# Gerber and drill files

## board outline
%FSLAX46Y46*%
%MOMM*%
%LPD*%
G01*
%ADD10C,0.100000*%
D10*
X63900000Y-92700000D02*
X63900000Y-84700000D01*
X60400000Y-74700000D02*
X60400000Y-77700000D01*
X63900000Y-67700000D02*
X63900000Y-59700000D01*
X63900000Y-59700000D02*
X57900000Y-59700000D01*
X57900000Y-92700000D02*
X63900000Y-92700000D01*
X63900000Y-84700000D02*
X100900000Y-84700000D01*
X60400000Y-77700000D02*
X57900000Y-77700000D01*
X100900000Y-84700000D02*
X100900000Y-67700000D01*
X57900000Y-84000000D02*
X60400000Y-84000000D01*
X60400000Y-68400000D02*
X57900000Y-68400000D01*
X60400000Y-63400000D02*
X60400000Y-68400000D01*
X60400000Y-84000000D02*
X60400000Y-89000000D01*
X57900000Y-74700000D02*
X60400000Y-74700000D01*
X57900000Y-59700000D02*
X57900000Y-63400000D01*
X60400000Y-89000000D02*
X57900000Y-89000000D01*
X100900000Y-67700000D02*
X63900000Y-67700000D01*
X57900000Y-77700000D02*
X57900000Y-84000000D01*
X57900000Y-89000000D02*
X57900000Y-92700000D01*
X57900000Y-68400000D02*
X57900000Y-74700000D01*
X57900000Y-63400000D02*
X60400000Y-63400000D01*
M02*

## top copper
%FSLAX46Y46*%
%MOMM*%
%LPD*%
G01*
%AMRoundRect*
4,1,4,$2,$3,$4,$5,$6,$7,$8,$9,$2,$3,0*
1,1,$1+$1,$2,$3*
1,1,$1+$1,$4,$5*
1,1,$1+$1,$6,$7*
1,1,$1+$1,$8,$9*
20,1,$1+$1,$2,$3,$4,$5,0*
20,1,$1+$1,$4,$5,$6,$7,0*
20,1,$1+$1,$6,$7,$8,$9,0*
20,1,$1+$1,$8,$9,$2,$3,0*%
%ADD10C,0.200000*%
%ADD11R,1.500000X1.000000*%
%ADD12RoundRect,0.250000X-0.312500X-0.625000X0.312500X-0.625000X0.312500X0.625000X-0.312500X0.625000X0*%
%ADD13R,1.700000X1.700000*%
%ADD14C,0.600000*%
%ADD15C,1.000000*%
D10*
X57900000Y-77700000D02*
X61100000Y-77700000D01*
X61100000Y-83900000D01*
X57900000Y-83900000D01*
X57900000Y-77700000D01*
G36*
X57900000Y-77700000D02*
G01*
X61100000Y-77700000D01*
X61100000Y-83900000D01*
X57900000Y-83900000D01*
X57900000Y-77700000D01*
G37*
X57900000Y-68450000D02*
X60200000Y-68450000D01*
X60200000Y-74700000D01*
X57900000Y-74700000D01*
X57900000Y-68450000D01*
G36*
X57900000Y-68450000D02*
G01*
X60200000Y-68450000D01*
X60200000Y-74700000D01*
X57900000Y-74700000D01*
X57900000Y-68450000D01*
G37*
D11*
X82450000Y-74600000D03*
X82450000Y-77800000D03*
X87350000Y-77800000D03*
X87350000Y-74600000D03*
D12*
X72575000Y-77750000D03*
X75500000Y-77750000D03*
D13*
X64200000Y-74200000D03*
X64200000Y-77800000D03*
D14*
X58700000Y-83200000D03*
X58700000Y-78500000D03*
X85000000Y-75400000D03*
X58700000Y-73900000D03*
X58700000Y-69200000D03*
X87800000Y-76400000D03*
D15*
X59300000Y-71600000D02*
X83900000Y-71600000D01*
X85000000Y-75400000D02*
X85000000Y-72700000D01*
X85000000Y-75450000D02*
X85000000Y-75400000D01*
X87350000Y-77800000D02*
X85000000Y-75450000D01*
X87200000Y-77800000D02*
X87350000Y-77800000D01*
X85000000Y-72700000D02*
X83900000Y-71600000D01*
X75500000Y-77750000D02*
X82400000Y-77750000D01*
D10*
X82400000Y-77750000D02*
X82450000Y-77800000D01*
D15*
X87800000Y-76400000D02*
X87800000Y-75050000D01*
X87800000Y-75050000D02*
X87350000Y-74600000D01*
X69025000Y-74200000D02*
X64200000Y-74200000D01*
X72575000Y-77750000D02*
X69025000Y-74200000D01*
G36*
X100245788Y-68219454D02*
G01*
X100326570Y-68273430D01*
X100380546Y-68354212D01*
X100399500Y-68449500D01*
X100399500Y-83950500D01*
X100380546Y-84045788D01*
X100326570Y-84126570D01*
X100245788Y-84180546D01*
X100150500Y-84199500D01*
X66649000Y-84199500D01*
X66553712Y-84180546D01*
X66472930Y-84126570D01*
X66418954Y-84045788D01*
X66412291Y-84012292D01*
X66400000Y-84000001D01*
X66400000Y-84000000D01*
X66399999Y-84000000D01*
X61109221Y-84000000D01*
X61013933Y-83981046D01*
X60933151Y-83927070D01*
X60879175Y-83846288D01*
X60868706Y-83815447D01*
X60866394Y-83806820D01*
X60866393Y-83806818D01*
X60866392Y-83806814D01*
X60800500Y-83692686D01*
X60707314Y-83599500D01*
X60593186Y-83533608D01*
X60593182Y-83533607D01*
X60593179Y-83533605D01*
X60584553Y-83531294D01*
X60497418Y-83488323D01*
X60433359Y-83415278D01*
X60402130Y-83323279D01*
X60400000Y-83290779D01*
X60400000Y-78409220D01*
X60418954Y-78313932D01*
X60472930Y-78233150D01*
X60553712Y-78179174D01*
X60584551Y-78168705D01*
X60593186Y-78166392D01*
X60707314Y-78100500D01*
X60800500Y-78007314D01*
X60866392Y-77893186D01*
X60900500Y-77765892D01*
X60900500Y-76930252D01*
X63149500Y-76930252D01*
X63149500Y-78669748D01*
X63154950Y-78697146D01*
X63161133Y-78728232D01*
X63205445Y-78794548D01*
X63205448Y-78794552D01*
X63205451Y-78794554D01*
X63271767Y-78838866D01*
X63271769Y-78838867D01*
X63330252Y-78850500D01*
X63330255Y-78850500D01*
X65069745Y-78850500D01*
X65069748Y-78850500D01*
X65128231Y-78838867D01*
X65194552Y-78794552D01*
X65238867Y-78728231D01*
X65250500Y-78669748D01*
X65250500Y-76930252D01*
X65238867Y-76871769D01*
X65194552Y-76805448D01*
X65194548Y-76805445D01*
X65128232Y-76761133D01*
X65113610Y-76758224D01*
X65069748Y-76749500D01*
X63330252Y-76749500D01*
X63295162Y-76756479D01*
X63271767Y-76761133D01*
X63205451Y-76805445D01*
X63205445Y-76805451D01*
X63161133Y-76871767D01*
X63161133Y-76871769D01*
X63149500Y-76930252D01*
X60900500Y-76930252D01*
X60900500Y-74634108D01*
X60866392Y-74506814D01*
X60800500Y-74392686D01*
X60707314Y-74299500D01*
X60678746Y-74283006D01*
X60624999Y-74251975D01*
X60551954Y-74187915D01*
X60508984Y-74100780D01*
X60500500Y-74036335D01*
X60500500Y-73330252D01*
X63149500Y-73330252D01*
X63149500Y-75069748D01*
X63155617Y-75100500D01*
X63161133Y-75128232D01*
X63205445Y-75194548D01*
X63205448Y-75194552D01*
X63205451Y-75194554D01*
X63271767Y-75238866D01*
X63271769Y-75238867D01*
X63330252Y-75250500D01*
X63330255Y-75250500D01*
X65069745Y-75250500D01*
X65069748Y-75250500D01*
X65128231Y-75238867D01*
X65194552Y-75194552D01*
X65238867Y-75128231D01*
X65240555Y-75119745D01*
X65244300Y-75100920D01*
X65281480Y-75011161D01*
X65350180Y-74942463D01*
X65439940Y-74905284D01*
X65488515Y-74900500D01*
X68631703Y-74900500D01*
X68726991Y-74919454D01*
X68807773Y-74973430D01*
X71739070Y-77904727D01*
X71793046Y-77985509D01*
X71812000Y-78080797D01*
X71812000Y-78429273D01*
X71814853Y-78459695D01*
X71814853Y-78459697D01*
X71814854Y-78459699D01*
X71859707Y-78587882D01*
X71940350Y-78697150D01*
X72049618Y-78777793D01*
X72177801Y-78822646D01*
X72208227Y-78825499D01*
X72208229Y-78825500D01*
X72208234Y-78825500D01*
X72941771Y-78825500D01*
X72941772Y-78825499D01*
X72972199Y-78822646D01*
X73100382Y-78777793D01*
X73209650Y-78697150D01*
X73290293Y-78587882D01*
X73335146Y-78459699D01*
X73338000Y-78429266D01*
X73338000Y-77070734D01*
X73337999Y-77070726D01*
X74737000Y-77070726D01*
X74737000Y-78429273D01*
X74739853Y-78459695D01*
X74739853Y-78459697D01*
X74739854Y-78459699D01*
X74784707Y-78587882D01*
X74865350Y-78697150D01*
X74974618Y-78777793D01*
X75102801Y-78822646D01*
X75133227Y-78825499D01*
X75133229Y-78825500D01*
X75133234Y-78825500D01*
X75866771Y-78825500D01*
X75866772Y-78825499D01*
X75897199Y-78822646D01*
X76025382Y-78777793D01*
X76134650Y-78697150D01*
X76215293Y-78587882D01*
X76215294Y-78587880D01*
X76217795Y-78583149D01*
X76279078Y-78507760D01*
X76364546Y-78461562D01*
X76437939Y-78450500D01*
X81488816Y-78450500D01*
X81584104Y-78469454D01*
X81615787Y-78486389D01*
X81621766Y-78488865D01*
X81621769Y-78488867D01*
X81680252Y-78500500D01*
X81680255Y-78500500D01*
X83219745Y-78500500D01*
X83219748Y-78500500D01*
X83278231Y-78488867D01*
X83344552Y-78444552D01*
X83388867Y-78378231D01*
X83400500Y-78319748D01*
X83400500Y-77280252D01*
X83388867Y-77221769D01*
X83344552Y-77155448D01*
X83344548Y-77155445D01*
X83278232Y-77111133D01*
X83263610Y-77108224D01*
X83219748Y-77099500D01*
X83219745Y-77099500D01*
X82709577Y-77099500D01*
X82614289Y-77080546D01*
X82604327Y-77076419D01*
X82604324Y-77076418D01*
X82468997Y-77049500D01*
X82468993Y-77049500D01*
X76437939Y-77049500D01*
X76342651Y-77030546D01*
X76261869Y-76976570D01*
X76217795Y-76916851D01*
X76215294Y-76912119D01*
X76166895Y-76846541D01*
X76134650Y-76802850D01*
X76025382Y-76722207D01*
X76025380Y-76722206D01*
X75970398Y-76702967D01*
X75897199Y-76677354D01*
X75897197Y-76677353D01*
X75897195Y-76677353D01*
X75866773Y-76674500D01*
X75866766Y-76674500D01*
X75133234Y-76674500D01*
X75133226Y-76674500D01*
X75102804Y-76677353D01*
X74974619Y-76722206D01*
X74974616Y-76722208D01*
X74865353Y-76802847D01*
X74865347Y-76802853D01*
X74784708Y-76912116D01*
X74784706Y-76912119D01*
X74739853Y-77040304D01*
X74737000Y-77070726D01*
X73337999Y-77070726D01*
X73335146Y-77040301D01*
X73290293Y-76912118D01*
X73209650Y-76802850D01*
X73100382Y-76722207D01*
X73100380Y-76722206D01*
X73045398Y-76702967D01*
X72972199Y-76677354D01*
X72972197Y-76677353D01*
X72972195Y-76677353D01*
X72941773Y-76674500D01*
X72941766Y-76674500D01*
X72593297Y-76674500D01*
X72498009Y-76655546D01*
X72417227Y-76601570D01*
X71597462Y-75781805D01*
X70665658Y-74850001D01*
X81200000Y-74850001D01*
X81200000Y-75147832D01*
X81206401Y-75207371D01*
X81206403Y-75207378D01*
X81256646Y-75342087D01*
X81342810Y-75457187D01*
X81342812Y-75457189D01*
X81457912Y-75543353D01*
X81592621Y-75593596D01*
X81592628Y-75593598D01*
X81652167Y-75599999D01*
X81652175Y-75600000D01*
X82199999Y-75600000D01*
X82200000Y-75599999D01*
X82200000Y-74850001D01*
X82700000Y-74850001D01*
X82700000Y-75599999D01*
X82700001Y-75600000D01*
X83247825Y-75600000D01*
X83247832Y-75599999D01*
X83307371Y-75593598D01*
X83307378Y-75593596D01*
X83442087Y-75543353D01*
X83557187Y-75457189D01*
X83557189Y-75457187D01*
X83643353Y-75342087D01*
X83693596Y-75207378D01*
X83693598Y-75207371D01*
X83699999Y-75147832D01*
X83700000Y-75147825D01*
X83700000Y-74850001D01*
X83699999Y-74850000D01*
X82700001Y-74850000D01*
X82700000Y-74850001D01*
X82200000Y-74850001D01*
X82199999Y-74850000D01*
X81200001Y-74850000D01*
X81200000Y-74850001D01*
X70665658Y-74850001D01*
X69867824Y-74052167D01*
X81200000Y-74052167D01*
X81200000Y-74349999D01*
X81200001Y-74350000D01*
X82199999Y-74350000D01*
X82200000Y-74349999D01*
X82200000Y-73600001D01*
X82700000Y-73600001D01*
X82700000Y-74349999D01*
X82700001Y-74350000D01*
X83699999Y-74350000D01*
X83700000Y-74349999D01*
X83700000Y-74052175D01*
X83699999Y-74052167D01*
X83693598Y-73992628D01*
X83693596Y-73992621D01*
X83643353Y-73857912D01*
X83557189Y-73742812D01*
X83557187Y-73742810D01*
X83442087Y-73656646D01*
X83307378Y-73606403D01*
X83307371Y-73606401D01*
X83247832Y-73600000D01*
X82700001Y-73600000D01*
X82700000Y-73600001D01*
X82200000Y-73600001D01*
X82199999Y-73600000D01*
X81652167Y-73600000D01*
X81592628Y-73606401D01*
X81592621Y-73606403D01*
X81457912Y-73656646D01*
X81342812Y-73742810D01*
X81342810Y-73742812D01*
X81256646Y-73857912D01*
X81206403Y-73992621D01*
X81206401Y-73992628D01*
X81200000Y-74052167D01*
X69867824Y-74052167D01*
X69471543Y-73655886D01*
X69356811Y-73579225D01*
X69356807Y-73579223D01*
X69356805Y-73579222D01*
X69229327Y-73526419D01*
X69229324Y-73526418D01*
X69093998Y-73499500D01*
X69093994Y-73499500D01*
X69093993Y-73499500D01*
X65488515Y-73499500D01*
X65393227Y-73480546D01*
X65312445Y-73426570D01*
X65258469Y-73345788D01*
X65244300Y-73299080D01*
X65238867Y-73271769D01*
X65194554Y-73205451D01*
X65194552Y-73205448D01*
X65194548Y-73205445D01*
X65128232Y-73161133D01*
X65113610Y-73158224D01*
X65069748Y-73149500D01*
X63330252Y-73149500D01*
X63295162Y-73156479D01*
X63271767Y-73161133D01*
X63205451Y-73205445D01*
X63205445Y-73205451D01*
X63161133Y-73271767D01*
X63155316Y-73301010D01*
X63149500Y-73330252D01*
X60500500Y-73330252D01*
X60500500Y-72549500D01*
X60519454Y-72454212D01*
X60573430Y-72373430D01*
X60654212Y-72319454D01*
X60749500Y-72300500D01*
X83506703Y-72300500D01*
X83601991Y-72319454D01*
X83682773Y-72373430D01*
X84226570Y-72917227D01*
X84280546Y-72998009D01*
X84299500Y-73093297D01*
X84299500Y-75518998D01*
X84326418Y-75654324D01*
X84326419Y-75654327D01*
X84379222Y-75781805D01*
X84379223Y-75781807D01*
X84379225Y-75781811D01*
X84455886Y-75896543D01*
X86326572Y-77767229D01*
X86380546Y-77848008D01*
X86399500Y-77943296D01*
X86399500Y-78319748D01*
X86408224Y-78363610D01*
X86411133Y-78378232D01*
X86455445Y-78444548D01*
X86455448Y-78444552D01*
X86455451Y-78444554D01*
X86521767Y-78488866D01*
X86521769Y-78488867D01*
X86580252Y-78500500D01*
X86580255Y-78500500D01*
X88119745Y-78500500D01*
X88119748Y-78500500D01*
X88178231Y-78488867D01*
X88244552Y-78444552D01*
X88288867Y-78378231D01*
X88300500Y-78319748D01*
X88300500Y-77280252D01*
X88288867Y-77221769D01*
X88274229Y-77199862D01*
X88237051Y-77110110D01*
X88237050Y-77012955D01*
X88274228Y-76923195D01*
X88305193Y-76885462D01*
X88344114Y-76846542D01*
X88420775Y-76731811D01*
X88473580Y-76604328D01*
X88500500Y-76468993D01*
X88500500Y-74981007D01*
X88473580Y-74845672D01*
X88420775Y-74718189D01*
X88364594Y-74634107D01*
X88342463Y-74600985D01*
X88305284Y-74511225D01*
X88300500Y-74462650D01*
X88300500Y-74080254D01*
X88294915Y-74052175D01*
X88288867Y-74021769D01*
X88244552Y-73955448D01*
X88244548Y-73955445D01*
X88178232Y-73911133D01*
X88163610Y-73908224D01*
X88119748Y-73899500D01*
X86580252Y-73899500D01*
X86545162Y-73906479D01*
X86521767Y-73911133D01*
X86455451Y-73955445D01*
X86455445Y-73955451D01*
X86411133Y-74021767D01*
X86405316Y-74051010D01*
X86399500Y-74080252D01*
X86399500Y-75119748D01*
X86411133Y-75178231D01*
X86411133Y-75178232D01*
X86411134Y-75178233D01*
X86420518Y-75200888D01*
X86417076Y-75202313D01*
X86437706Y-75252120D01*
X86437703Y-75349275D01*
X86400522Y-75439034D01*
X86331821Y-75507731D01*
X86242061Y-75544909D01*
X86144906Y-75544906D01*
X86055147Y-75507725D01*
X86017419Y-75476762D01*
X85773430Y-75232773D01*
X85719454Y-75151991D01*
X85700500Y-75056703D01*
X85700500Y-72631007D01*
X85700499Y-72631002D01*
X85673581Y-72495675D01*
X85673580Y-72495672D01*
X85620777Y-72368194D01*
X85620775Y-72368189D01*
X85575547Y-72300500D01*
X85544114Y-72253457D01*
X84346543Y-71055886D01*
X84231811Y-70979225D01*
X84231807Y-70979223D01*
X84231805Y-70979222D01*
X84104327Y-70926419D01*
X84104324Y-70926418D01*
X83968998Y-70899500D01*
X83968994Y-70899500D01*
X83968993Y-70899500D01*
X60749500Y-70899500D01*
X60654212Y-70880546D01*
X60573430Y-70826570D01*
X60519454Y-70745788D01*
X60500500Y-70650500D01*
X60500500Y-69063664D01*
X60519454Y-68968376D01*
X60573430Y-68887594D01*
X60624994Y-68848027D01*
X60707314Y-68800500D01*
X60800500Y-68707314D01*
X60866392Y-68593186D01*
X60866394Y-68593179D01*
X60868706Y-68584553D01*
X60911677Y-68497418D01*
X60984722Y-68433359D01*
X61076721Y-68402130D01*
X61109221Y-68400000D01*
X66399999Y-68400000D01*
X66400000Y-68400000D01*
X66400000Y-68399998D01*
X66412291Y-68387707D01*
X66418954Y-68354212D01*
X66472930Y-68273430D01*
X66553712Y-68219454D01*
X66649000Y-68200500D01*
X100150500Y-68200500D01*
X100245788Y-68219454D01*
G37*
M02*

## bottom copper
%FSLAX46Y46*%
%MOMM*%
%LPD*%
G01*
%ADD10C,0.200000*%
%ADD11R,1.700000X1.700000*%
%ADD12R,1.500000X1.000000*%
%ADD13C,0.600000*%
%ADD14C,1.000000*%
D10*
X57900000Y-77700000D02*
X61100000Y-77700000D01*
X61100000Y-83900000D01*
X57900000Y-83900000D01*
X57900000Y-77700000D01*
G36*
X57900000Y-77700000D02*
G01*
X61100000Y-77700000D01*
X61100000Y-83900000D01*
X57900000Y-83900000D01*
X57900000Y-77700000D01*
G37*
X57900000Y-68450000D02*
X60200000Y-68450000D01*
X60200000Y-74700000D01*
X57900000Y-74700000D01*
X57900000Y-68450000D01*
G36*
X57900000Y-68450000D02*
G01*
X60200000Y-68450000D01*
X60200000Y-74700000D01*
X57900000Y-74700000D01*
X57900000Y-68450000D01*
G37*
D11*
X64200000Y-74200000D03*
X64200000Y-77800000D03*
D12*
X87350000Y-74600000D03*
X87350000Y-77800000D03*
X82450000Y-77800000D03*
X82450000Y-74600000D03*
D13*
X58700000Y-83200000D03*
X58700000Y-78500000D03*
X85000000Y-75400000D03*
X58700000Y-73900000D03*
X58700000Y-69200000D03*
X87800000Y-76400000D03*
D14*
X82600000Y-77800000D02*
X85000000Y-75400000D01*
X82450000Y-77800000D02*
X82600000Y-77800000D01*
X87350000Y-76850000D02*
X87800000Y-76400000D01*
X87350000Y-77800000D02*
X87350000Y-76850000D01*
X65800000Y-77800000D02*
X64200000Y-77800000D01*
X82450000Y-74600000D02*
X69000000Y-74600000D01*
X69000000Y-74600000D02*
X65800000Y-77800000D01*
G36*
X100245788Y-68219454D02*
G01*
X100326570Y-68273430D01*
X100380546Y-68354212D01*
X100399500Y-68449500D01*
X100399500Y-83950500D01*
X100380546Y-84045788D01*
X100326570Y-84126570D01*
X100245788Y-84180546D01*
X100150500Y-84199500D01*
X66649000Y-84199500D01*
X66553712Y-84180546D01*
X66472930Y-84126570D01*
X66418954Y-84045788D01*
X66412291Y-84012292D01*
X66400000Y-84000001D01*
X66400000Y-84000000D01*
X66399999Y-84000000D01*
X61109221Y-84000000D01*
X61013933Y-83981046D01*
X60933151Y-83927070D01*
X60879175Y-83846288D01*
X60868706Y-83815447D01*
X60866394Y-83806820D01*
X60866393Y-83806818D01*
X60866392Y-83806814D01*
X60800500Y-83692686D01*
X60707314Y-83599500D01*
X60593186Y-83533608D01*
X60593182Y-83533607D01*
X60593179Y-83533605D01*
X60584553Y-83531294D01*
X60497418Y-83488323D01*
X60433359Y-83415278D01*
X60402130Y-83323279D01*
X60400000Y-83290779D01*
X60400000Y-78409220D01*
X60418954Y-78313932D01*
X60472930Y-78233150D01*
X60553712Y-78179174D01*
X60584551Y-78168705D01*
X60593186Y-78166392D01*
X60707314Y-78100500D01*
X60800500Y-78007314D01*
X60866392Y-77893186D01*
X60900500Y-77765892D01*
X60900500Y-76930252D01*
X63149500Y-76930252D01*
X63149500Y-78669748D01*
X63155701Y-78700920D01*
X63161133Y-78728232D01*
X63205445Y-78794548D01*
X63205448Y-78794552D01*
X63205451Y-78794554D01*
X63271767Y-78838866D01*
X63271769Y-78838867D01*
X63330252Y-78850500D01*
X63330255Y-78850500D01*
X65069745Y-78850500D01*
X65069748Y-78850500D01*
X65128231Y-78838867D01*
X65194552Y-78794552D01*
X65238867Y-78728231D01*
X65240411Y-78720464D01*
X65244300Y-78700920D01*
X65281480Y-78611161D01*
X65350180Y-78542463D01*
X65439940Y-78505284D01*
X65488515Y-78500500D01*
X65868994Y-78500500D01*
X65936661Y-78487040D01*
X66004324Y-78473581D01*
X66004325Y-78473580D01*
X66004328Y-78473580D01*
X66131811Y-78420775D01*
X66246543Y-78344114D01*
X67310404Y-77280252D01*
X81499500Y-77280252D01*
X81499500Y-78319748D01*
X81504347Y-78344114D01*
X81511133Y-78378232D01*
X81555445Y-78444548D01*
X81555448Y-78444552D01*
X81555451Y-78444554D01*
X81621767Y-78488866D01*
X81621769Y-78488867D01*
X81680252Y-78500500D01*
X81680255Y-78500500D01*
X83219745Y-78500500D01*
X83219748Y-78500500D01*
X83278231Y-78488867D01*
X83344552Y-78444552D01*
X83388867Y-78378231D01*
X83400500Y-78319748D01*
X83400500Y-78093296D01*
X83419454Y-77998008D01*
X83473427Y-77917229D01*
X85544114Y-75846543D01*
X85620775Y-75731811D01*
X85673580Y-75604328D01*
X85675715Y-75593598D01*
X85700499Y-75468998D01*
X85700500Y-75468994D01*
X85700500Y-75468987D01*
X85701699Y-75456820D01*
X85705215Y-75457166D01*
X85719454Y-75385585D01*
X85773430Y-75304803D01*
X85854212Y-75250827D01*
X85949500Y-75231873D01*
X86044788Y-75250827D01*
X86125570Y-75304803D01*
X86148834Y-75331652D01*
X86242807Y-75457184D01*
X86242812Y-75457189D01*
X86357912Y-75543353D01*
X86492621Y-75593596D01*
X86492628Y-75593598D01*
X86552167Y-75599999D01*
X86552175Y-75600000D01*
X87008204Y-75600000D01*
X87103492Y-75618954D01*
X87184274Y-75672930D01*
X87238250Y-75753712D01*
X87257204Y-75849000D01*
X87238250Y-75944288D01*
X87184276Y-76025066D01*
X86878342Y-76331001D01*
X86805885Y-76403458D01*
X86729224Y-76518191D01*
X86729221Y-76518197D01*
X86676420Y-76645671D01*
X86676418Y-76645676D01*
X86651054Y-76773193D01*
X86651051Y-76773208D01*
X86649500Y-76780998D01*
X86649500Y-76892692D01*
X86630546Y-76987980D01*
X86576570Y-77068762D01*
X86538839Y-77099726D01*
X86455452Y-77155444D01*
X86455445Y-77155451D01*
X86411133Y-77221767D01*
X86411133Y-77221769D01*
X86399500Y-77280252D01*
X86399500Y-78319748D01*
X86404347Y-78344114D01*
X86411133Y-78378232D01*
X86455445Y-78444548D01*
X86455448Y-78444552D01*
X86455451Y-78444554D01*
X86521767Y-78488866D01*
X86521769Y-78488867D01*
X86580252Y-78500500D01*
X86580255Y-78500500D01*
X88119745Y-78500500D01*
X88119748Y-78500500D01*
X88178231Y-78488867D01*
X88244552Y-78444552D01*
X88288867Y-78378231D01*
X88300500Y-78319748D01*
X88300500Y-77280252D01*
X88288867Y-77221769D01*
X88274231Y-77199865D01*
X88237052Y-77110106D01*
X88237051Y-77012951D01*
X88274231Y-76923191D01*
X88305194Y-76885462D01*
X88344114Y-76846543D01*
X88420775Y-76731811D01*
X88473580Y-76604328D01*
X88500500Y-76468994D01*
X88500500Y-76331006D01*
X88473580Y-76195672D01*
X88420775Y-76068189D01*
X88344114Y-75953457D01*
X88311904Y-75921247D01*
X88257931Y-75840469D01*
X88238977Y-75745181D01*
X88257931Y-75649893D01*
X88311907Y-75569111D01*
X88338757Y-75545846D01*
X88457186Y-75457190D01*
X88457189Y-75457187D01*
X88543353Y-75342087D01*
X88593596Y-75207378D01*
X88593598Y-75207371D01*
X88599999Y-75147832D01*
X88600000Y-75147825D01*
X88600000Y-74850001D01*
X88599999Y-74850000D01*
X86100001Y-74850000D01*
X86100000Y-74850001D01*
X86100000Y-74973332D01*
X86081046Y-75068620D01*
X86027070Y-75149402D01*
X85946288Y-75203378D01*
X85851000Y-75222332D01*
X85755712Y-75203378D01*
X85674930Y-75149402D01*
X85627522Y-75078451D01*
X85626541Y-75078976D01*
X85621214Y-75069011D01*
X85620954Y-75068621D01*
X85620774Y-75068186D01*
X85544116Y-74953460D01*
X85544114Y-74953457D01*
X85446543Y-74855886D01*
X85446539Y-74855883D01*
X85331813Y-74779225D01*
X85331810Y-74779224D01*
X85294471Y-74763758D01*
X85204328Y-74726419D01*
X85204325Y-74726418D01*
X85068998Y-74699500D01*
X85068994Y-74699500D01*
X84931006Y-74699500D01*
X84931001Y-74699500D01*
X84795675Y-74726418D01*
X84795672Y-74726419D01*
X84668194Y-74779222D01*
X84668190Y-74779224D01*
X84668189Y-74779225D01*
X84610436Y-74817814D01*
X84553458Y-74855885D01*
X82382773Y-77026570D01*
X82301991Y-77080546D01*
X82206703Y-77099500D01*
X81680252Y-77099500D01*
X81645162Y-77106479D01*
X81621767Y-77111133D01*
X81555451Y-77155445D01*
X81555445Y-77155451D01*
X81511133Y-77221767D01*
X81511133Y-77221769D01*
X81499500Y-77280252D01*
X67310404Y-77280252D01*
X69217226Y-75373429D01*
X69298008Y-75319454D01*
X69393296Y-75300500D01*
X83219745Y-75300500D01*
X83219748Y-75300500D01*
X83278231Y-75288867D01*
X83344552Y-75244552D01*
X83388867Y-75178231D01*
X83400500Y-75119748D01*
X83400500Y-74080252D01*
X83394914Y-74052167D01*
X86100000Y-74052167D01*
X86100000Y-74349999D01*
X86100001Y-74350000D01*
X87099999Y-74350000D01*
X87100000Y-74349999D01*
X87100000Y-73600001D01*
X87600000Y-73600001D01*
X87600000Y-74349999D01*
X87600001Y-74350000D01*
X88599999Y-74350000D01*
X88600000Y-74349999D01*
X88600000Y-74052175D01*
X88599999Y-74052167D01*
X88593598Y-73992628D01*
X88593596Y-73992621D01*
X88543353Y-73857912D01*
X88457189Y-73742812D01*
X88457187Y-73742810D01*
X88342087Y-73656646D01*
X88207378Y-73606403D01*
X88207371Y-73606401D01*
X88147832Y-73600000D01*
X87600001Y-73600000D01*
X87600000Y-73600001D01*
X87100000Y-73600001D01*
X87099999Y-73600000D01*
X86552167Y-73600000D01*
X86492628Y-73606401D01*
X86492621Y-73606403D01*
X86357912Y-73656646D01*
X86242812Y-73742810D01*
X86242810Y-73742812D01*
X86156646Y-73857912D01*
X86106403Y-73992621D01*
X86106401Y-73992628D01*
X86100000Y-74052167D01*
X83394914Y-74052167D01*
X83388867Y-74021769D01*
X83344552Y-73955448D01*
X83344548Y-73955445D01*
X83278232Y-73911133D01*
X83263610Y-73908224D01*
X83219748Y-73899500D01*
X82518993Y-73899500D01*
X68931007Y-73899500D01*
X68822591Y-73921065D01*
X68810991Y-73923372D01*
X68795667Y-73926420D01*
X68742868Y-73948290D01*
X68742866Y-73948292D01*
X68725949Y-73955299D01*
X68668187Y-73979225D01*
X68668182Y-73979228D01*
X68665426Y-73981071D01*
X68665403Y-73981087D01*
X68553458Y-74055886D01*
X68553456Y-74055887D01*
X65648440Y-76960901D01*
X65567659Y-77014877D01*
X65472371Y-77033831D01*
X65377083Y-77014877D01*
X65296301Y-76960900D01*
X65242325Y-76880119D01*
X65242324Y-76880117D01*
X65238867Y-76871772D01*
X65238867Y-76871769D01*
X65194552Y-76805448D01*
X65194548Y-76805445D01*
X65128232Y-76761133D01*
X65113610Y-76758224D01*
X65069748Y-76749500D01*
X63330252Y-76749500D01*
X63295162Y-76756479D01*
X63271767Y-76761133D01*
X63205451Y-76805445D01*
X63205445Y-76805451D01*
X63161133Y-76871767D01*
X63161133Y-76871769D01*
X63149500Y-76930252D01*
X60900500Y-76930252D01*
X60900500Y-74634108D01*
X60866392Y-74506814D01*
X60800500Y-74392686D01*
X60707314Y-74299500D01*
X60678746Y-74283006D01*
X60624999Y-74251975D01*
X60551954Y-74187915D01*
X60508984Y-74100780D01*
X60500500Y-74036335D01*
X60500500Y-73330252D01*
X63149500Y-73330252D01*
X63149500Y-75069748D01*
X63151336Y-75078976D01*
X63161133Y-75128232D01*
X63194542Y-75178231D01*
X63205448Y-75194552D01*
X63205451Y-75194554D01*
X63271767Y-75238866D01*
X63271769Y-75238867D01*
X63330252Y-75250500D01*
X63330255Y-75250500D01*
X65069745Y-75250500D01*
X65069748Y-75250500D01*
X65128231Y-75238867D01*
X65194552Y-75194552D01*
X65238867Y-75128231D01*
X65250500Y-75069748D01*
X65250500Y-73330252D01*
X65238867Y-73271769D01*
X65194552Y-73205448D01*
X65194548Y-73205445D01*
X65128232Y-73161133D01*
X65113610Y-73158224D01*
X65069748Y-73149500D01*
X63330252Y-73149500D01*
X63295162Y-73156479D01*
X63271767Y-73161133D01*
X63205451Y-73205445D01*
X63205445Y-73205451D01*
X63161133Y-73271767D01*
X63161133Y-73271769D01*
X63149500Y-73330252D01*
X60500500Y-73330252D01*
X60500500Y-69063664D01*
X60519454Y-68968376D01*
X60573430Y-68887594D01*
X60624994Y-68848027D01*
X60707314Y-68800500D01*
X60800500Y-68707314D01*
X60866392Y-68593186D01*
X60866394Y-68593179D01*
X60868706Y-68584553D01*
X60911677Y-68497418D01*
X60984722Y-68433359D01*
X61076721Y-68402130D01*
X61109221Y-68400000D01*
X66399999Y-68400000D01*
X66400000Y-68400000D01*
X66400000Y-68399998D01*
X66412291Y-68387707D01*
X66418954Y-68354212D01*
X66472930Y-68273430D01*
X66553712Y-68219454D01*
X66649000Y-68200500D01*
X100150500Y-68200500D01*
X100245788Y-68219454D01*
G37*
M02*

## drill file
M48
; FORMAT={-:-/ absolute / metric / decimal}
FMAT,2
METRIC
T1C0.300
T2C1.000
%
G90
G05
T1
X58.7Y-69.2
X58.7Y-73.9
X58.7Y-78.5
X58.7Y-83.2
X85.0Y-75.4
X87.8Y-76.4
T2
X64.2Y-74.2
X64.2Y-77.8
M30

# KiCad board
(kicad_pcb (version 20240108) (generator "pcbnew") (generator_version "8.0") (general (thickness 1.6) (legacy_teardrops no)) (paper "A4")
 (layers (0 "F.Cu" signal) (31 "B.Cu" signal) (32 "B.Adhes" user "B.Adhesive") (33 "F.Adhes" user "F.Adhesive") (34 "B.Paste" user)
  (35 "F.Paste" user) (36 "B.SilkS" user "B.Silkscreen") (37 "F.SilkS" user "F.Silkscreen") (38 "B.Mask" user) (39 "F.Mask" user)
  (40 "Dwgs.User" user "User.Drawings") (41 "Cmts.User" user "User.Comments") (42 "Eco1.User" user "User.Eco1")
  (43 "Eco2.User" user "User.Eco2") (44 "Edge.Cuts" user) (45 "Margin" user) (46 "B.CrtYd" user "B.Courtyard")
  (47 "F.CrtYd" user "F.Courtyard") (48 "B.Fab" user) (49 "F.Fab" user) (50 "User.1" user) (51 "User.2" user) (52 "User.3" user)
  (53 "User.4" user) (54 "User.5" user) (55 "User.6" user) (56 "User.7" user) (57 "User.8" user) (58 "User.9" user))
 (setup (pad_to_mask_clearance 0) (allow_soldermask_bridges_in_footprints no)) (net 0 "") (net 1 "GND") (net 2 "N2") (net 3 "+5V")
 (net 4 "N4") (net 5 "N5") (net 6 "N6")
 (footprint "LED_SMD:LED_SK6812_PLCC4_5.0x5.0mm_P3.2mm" (layer "F.Cu") (at 84.9 76.2 180)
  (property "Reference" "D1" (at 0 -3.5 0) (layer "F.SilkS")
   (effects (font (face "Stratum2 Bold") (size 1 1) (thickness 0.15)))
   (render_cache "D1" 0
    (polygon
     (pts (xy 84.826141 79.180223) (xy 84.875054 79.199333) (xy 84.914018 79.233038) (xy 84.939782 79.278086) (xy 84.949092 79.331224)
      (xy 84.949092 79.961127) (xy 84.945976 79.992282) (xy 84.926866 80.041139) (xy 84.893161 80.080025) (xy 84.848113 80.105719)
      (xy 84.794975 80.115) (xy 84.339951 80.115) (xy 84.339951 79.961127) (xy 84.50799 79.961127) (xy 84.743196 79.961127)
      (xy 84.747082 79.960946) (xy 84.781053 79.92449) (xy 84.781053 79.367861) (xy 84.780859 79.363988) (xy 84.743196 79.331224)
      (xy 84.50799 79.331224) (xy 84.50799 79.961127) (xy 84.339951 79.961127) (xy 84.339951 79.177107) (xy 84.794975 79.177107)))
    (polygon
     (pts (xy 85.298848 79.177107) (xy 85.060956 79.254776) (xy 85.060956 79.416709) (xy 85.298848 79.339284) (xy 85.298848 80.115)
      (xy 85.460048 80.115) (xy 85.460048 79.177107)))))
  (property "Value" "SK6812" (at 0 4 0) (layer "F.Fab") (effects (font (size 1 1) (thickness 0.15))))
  (pad "1" smd rect (at 2.45 1.6 180) (size 1.5 1) (layers "F.Cu" "F.Paste" "F.Mask") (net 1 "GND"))
  (pad "2" smd rect (at 2.45 -1.6 180) (size 1.5 1) (layers "F.Cu" "F.Paste" "F.Mask") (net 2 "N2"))
  (pad "3" smd rect (at -2.45 -1.6 180) (size 1.5 1) (layers "F.Cu" "F.Paste" "F.Mask") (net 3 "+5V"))
  (pad "4" smd rect (at -2.45 1.6 180) (size 1.5 1) (layers "F.Cu" "F.Paste" "F.Mask") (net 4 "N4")))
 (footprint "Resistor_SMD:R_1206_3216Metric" (layer "F.Cu") (at 74.0375 77.75)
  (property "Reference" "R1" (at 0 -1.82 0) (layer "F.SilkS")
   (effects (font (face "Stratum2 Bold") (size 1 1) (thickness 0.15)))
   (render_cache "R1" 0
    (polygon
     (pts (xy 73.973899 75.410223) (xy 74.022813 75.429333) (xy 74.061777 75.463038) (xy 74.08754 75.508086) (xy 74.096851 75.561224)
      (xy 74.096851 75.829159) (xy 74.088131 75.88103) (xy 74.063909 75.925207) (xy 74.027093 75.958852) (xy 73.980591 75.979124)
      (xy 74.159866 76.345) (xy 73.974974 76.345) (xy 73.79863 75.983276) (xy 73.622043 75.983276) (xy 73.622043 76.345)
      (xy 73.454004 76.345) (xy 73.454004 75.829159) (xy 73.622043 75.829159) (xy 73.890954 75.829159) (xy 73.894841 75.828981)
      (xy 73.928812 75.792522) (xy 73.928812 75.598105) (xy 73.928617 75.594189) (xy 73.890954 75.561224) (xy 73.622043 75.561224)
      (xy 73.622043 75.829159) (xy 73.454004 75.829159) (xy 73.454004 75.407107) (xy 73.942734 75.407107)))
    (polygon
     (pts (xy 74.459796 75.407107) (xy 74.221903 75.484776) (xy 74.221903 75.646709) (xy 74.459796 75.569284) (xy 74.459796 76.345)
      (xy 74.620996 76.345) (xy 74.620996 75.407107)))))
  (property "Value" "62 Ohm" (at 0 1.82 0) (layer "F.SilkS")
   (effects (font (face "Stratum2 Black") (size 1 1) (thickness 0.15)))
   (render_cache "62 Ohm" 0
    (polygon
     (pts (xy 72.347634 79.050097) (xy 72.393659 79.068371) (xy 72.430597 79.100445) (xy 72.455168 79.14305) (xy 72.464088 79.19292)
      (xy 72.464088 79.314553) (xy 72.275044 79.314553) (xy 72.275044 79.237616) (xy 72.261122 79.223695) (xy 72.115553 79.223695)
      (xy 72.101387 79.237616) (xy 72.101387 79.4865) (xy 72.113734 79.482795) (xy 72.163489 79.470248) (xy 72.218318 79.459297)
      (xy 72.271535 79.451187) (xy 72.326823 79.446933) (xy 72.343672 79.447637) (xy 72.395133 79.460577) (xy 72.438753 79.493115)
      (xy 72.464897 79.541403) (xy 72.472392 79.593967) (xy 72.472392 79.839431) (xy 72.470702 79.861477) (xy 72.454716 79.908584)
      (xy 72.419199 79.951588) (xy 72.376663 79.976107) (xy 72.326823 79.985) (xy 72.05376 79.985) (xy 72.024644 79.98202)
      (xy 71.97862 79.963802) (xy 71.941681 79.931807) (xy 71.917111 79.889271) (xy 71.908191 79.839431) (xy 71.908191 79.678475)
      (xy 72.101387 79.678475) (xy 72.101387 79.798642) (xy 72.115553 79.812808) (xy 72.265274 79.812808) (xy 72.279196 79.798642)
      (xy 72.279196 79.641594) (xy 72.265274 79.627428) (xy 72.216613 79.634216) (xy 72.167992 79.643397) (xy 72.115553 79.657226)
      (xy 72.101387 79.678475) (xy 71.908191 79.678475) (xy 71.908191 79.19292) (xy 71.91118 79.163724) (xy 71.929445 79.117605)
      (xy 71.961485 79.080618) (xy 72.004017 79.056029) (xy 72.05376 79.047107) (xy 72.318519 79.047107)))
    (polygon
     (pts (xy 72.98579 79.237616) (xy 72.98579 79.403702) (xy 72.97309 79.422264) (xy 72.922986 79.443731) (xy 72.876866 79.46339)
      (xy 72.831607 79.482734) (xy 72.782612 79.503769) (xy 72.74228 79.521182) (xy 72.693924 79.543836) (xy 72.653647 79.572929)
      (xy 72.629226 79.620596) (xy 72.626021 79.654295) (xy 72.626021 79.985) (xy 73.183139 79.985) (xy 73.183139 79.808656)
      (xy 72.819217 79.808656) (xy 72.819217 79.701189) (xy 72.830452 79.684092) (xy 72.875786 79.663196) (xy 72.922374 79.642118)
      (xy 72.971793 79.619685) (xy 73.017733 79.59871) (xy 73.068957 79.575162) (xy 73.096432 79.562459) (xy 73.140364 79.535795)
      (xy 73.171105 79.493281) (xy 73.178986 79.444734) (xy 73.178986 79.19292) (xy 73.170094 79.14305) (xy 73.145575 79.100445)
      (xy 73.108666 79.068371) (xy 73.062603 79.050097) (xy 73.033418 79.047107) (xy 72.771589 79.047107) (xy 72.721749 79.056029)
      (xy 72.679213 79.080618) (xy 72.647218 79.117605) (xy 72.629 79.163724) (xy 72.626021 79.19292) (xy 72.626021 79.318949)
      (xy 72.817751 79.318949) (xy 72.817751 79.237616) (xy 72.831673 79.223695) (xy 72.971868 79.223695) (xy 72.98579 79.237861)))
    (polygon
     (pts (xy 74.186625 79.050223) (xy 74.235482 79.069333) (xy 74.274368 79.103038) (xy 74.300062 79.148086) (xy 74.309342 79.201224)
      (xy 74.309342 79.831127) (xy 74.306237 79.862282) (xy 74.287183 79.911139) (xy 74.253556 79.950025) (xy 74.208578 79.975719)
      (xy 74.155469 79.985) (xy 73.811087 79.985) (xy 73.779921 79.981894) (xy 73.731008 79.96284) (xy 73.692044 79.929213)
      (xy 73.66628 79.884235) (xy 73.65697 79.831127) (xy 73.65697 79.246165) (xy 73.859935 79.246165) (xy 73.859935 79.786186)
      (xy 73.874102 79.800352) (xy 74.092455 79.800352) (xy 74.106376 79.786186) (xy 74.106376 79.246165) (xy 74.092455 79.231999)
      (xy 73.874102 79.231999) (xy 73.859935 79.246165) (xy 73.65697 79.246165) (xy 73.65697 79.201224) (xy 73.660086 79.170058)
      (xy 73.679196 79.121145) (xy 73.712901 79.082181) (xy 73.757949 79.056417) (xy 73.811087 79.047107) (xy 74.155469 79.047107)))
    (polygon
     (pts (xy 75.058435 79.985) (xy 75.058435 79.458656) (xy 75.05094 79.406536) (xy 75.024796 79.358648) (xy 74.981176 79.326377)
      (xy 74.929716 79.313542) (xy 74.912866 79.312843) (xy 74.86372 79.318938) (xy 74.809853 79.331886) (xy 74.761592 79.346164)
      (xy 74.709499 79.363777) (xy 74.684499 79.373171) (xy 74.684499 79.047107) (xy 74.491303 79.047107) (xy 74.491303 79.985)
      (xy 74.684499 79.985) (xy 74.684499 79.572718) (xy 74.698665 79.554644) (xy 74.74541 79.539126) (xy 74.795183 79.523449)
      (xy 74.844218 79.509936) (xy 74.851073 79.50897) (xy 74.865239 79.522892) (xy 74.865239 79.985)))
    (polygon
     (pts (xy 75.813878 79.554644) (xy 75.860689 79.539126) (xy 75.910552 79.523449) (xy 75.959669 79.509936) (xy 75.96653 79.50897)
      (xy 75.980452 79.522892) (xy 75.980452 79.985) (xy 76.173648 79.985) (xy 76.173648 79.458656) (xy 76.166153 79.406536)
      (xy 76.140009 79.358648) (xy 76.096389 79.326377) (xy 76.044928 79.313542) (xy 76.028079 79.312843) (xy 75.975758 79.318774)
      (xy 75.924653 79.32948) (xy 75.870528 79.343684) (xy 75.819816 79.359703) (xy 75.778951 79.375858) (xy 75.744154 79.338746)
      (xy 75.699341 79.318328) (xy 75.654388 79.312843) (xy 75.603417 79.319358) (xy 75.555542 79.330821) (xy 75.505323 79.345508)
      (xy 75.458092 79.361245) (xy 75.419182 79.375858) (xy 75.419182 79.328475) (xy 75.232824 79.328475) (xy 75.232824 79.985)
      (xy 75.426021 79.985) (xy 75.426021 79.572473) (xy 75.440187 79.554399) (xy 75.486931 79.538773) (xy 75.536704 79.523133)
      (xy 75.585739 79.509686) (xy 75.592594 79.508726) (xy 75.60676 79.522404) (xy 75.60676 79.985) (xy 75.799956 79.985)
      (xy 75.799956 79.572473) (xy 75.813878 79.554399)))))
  (pad "1" smd roundrect (at -1.4625 0) (size 1.125 1.75) (layers "F.Cu" "F.Paste" "F.Mask") (roundrect_rratio 0.222222) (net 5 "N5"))
  (pad "2" smd roundrect (at 1.4625 0) (size 1.125 1.75) (layers "F.Cu" "F.Paste" "F.Mask") (roundrect_rratio 0.222222) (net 2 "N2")))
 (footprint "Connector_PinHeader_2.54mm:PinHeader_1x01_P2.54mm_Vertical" (layer "F.Cu") (at 64.2 74.2)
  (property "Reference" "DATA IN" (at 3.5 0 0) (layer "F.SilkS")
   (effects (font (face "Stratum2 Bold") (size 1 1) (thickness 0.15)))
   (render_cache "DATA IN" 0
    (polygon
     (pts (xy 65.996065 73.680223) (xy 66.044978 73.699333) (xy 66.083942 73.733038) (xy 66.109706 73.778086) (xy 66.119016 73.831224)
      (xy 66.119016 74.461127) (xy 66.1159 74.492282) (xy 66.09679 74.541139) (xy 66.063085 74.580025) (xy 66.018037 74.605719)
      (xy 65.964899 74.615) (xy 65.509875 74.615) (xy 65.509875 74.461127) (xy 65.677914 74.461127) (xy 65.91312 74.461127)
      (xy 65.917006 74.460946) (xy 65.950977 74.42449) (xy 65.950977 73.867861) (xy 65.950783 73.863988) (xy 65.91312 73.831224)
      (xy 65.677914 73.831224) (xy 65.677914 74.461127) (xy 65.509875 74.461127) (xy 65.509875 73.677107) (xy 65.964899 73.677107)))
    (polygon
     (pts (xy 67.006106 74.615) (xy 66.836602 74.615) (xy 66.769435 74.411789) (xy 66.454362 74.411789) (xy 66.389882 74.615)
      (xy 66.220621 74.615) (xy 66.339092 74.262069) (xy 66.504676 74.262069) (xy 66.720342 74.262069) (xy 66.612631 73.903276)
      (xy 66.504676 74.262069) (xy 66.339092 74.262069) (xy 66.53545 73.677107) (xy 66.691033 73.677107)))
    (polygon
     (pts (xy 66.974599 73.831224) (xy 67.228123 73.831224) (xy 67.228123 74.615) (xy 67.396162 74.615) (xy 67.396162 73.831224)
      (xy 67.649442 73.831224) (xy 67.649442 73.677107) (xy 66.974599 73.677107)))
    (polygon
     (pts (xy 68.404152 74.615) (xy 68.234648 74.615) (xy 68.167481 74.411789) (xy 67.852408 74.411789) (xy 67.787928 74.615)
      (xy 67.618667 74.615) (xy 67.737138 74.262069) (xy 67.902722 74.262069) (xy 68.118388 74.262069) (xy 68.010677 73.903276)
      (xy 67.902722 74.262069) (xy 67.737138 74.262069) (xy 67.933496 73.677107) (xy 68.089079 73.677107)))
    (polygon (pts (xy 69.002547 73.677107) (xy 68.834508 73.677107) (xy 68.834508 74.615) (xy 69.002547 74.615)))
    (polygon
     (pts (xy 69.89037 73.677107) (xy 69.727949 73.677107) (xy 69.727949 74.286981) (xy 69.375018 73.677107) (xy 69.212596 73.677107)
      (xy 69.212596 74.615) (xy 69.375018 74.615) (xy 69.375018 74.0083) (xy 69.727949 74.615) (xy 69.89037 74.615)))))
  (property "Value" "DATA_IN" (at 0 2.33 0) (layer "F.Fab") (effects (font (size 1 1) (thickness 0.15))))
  (pad "1" thru_hole rect (at 0 0) (size 1.7 1.7) (drill 1) (layers "*.Cu" "*.Mask") (remove_unused_layers no) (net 5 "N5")))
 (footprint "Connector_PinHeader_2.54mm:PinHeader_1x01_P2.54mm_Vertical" (layer "F.Cu") (at 64.2 77.8)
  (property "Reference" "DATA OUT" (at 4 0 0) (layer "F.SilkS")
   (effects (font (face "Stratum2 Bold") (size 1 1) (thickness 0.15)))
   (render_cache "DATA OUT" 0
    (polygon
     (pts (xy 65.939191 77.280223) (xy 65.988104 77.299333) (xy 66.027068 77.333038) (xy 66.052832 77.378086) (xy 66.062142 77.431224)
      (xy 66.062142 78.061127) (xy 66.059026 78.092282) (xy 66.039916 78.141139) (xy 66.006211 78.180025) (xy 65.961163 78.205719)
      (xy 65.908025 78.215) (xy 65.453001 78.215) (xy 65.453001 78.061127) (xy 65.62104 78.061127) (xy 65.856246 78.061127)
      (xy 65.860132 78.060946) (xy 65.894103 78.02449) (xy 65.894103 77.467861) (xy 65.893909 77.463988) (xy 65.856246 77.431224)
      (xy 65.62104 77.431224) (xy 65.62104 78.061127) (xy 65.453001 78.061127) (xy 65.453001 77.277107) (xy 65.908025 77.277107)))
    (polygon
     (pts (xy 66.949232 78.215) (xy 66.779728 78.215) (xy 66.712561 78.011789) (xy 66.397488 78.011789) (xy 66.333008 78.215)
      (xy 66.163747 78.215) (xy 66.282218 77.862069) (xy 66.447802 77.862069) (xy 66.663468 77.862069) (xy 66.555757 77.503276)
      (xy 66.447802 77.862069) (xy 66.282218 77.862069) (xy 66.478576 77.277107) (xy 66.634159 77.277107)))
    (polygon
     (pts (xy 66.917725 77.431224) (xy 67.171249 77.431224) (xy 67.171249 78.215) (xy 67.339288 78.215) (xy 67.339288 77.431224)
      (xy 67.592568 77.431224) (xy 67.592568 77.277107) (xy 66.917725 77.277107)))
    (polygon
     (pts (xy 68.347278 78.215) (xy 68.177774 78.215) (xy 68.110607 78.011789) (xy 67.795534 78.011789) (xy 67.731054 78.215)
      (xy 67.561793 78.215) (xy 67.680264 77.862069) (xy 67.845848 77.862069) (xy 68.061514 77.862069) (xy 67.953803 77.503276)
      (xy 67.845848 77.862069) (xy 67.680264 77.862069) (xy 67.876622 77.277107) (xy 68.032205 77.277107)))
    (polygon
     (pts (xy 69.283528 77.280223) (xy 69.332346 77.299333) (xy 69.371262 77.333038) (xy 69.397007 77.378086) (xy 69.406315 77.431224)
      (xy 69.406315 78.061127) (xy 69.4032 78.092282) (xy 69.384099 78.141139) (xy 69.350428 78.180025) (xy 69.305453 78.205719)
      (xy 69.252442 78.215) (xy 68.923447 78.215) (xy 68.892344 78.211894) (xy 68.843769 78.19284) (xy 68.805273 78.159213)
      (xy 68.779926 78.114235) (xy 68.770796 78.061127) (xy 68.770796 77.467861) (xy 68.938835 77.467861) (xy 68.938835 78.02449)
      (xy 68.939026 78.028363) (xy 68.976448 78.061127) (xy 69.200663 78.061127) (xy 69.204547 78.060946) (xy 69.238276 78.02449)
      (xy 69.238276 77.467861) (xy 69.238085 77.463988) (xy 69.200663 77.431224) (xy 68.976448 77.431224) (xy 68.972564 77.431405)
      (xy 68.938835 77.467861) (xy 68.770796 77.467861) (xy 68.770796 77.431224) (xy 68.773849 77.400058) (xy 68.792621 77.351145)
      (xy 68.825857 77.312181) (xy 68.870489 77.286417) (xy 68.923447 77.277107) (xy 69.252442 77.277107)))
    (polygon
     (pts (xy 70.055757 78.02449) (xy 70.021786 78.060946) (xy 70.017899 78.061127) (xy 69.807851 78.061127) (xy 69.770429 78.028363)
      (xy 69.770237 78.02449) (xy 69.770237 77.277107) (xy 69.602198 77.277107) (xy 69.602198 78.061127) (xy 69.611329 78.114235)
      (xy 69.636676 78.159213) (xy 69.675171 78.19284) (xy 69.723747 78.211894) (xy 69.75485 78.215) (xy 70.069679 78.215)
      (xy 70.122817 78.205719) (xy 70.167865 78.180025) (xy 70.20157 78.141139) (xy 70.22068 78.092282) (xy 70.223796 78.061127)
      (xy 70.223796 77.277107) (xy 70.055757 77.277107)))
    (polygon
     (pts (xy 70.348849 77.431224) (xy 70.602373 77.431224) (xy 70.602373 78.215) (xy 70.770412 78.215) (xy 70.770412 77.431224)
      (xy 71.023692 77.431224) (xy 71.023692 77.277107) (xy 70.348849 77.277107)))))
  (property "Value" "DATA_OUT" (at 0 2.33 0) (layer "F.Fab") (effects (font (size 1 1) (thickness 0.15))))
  (pad "1" thru_hole rect (at 0 0) (size 1.7 1.7) (drill 1) (layers "*.Cu" "*.Mask") (remove_unused_layers no) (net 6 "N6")))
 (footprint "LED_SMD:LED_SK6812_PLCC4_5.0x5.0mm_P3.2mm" (layer "B.Cu") (at 84.9 76.2)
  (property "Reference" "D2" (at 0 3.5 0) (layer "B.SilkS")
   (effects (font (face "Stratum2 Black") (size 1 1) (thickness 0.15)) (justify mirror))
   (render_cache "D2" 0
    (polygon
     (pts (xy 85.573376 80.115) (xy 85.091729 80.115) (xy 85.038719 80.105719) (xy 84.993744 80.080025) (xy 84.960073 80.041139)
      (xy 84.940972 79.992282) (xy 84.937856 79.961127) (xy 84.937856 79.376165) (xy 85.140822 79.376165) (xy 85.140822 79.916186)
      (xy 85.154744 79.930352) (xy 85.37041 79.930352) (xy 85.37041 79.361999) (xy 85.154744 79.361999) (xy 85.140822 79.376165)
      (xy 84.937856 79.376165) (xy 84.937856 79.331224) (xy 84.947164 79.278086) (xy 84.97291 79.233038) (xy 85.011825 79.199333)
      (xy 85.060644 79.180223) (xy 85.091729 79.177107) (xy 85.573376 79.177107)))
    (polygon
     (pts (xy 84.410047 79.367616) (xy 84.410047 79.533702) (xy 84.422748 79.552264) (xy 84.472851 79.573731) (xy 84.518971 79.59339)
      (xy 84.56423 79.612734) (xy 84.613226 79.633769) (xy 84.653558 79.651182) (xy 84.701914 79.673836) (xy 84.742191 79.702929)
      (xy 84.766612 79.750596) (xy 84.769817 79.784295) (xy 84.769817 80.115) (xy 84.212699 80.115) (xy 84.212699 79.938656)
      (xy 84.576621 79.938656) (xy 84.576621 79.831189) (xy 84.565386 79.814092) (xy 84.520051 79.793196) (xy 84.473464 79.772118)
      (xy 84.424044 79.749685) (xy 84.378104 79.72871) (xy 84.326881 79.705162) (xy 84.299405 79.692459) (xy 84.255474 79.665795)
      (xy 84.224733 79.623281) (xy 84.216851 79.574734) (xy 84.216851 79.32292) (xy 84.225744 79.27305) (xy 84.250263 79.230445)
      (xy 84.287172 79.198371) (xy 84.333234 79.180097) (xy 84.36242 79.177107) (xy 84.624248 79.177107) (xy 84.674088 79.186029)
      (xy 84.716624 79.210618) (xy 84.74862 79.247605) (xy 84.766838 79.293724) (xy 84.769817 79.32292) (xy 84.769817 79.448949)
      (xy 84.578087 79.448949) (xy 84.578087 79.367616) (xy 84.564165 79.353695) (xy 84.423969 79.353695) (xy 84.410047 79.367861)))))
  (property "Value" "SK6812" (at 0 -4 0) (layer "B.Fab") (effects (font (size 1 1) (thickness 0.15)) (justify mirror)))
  (pad "1" smd rect (at 2.45 -1.6) (size 1.5 1) (layers "B.Cu" "B.Paste" "B.Mask") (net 1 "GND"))
  (pad "2" smd rect (at 2.45 1.6) (size 1.5 1) (layers "B.Cu" "B.Paste" "B.Mask") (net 4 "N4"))
  (pad "3" smd rect (at -2.45 1.6) (size 1.5 1) (layers "B.Cu" "B.Paste" "B.Mask") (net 3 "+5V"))
  (pad "4" smd rect (at -2.45 -1.6) (size 1.5 1) (layers "B.Cu" "B.Paste" "B.Mask") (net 6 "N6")))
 (gr_rect (start 57.9 77.7) (end 61.1 83.9) (stroke (width 0.2) (type default)) (fill solid) (layer "F.Cu") (net 1))
 (gr_rect (start 57.9 68.45) (end 60.2 74.7) (stroke (width 0.2) (type default)) (fill solid) (layer "F.Cu") (net 3))
 (gr_rect (start 57.9 77.7) (end 61.1 83.9) (stroke (width 0.2) (type default)) (fill solid) (layer "B.Cu") (net 1))
 (gr_rect (start 57.9 68.45) (end 60.2 74.7) (stroke (width 0.2) (type default)) (fill solid) (layer "B.Cu") (net 3))
 (gr_line (start 63.9 92.7) (end 63.9 84.7) (stroke (width 0.1) (type default)) (layer "Edge.Cuts"))
 (gr_line (start 60.4 74.7) (end 60.4 77.7) (stroke (width 0.1) (type default)) (layer "Edge.Cuts"))
 (gr_line (start 63.9 67.7) (end 63.9 59.7) (stroke (width 0.1) (type default)) (layer "Edge.Cuts"))
 (gr_line (start 63.9 59.7) (end 57.9 59.7) (stroke (width 0.1) (type default)) (layer "Edge.Cuts"))
 (gr_line (start 57.9 92.7) (end 63.9 92.7) (stroke (width 0.1) (type default)) (layer "Edge.Cuts"))
 (gr_line (start 63.9 84.7) (end 100.9 84.7) (stroke (width 0.1) (type default)) (layer "Edge.Cuts"))
 (gr_line (start 60.4 77.7) (end 57.9 77.7) (stroke (width 0.1) (type default)) (layer "Edge.Cuts"))
 (gr_line (start 100.9 84.7) (end 100.9 67.7) (stroke (width 0.1) (type default)) (layer "Edge.Cuts"))
 (gr_line (start 57.9 84) (end 60.4 84) (stroke (width 0.1) (type default)) (layer "Edge.Cuts"))
 (gr_line (start 60.4 68.4) (end 57.9 68.4) (stroke (width 0.1) (type default)) (layer "Edge.Cuts"))
 (gr_line (start 60.4 63.4) (end 60.4 68.4) (stroke (width 0.1) (type default)) (layer "Edge.Cuts"))
 (gr_line (start 60.4 84) (end 60.4 89) (stroke (width 0.1) (type default)) (layer "Edge.Cuts"))
 (gr_line (start 57.9 74.7) (end 60.4 74.7) (stroke (width 0.1) (type default)) (layer "Edge.Cuts"))
 (gr_line (start 57.9 59.7) (end 57.9 63.4) (stroke (width 0.1) (type default)) (layer "Edge.Cuts"))
 (gr_line (start 60.4 89) (end 57.9 89) (stroke (width 0.1) (type default)) (layer "Edge.Cuts"))
 (gr_line (start 100.9 67.7) (end 63.9 67.7) (stroke (width 0.1) (type default)) (layer "Edge.Cuts"))
 (gr_line (start 57.9 77.7) (end 57.9 84) (stroke (width 0.1) (type default)) (layer "Edge.Cuts"))
 (gr_line (start 57.9 89) (end 57.9 92.7) (stroke (width 0.1) (type default)) (layer "Edge.Cuts"))
 (gr_line (start 57.9 68.4) (end 57.9 74.7) (stroke (width 0.1) (type default)) (layer "Edge.Cuts"))
 (gr_line (start 57.9 63.4) (end 60.4 63.4) (stroke (width 0.1) (type default)) (layer "Edge.Cuts"))
 (via (at 58.7 83.2) (size 0.6) (drill 0.3) (layers "F.Cu" "B.Cu") (free yes) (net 1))
 (via (at 58.7 78.5) (size 0.6) (drill 0.3) (layers "F.Cu" "B.Cu") (free yes) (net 1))
 (segment (start 59.3 71.6) (end 83.9 71.6) (width 1) (layer "F.Cu") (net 3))
 (segment (start 85 75.4) (end 85 72.7) (width 1) (layer "F.Cu") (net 3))
 (segment (start 85 75.45) (end 85 75.4) (width 1) (layer "F.Cu") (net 3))
 (segment (start 87.35 77.8) (end 85 75.45) (width 1) (layer "F.Cu") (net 3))
 (segment (start 87.2 77.8) (end 87.35 77.8) (width 1) (layer "F.Cu") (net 3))
 (segment (start 85 72.7) (end 83.9 71.6) (width 1) (layer "F.Cu") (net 3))
 (via (at 85 75.4) (size 0.6) (drill 0.3) (layers "F.Cu" "B.Cu") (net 3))
 (via (at 58.7 73.9) (size 0.6) (drill 0.3) (layers "F.Cu" "B.Cu") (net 3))
 (via (at 58.7 69.2) (size 0.6) (drill 0.3) (layers "F.Cu" "B.Cu") (free yes) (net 3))
 (segment (start 82.6 77.8) (end 85 75.4) (width 1) (layer "B.Cu") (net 3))
 (segment (start 82.45 77.8) (end 82.6 77.8) (width 1) (layer "B.Cu") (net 3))
 (segment (start 75.5 77.75) (end 82.4 77.75) (width 1) (layer "F.Cu") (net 2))
 (segment (start 82.4 77.75) (end 82.45 77.8) (width 0.2) (layer "F.Cu") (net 2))
 (segment (start 87.8 76.4) (end 87.8 75.05) (width 1) (layer "F.Cu") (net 4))
 (segment (start 87.8 75.05) (end 87.35 74.6) (width 1) (layer "F.Cu") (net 4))
 (via (at 87.8 76.4) (size 0.6) (drill 0.3) (layers "F.Cu" "B.Cu") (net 4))
 (segment (start 87.35 76.85) (end 87.8 76.4) (width 1) (layer "B.Cu") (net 4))
 (segment (start 87.35 77.8) (end 87.35 76.85) (width 1) (layer "B.Cu") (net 4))
 (segment (start 65.8 77.8) (end 64.2 77.8) (width 1) (layer "B.Cu") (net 6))
 (segment (start 82.45 74.6) (end 69 74.6) (width 1) (layer "B.Cu") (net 6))
 (segment (start 69 74.6) (end 65.8 77.8) (width 1) (layer "B.Cu") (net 6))
 (segment (start 69.025 74.2) (end 64.2 74.2) (width 1) (layer "F.Cu") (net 5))
 (segment (start 72.575 77.75) (end 69.025 74.2) (width 1) (layer "F.Cu") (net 5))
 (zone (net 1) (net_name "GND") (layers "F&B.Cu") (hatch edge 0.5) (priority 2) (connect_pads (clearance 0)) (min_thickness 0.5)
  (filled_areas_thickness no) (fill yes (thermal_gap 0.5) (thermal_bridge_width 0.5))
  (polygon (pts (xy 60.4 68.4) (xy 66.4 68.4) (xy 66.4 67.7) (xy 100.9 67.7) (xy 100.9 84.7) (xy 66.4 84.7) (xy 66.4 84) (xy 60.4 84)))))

